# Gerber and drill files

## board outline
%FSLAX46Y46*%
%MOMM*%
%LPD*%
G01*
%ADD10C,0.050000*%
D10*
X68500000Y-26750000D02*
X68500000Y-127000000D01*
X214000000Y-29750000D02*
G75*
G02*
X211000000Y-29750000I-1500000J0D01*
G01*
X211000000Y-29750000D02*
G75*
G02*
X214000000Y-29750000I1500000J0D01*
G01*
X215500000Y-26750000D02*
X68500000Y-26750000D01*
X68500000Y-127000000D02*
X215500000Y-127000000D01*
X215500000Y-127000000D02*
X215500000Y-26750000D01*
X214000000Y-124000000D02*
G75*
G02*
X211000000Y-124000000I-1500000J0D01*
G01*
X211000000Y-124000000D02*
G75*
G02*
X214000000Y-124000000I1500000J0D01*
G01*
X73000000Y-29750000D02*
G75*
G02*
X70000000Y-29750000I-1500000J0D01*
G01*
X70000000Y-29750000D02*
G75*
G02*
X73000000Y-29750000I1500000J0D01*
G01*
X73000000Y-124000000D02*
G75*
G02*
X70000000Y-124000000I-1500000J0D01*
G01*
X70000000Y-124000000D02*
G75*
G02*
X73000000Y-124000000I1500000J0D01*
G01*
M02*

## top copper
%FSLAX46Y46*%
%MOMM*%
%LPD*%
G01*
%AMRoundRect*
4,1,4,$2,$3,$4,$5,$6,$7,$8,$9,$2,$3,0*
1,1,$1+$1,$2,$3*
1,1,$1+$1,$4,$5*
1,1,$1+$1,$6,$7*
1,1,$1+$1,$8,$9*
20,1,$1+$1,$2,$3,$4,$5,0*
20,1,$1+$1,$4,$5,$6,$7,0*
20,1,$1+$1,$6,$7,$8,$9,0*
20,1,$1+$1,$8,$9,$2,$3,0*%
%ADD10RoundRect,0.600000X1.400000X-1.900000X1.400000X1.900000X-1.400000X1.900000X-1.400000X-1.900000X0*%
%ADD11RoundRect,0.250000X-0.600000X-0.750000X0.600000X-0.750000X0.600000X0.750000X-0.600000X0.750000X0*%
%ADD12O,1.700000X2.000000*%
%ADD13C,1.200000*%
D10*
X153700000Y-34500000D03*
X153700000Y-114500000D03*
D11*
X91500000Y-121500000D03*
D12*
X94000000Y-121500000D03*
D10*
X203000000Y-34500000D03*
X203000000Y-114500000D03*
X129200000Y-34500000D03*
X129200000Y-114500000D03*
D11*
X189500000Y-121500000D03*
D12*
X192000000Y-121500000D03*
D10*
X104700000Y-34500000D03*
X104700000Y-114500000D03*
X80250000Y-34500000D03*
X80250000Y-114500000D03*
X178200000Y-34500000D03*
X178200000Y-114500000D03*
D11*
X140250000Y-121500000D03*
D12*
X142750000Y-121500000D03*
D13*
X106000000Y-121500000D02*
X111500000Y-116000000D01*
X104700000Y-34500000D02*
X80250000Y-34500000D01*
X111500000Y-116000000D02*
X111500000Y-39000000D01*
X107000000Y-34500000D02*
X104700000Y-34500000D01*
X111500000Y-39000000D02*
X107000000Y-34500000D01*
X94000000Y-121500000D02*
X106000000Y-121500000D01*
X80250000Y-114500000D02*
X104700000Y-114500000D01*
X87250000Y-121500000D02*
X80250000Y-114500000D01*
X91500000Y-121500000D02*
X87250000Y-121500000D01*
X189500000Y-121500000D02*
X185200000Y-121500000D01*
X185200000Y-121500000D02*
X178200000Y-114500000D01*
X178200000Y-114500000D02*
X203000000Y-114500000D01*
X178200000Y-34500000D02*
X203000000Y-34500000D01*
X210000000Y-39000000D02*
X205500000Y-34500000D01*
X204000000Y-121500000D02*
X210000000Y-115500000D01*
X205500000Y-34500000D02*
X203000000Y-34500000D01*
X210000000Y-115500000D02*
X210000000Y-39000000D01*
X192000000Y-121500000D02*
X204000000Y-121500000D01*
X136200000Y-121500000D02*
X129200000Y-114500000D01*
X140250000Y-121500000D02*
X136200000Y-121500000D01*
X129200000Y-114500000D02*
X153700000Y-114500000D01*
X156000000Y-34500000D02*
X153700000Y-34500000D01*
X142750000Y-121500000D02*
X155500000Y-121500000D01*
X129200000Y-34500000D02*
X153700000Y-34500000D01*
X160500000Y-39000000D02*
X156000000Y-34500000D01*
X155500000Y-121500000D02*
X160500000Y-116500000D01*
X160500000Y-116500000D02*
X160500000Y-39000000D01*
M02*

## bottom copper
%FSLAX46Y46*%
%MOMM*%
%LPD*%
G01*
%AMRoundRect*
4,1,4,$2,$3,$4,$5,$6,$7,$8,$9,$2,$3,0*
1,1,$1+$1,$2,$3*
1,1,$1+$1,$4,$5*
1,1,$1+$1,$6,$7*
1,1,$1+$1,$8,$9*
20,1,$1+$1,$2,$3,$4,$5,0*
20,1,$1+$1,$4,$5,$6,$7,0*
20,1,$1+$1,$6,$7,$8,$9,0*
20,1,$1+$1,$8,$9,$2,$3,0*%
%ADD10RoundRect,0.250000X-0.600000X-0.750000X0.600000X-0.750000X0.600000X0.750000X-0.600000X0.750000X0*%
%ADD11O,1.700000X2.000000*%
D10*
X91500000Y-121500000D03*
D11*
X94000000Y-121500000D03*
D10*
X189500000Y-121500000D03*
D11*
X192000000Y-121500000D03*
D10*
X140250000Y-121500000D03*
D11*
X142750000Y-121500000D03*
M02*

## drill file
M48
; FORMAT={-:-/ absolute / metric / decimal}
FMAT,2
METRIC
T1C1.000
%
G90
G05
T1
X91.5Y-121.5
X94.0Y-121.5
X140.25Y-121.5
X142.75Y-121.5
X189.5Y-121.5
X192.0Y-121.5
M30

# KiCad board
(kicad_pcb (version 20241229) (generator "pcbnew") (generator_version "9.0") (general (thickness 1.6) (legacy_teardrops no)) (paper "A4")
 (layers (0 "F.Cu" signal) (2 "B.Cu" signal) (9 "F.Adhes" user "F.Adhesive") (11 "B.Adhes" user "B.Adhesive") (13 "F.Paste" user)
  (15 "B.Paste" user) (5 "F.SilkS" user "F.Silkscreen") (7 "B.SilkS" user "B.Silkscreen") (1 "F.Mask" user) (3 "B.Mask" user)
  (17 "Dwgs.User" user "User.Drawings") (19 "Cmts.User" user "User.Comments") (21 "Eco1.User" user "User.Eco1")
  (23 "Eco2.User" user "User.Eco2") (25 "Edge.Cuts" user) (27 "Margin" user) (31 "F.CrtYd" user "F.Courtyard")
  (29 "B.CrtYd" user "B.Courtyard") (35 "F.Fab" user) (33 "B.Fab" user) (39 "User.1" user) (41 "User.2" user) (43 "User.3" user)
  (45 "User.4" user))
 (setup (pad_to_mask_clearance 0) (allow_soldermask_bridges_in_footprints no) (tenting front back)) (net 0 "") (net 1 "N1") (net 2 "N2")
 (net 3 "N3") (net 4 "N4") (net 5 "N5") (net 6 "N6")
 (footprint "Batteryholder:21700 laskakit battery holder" (layer "F.Cu") (at 153.7 79.5)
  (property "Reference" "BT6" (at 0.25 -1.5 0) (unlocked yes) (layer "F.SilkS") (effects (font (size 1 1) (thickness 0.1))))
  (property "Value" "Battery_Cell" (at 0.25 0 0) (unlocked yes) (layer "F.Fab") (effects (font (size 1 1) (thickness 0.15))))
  (pad "1" smd roundrect (at 0 -45 90) (size 5 4) (layers "F.Cu" "F.Mask" "F.Paste") (roundrect_rratio 0.15) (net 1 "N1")
   (thermal_bridge_angle 45))
  (pad "2" smd roundrect (at 0 35 90) (size 5 4) (layers "F.Cu" "F.Mask" "F.Paste") (roundrect_rratio 0.15) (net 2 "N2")
   (thermal_bridge_angle 45)))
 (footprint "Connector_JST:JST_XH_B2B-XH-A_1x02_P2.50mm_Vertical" (layer "F.Cu") (at 91.5 121.5)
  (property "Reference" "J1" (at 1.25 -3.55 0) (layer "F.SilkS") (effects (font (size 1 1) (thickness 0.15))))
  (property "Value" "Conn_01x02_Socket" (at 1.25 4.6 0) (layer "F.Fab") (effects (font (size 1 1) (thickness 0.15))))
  (pad "1" thru_hole roundrect (at 0 0) (size 1.7 2) (drill 1) (layers "*.Cu" "*.Mask") (remove_unused_layers no)
   (roundrect_rratio 0.147059) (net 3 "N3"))
  (pad "2" thru_hole oval (at 2.5 0) (size 1.7 2) (drill 1) (layers "*.Cu" "*.Mask") (remove_unused_layers no) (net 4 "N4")))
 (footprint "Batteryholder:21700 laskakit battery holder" (layer "F.Cu") (at 203 79.5)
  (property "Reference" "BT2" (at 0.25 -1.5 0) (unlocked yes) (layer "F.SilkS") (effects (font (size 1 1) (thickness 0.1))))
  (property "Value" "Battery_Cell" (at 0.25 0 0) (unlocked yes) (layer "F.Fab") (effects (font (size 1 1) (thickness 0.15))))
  (pad "1" smd roundrect (at 0 -45 90) (size 5 4) (layers "F.Cu" "F.Mask" "F.Paste") (roundrect_rratio 0.15) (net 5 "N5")
   (thermal_bridge_angle 45))
  (pad "2" smd roundrect (at 0 35 90) (size 5 4) (layers "F.Cu" "F.Mask" "F.Paste") (roundrect_rratio 0.15) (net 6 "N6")
   (thermal_bridge_angle 45)))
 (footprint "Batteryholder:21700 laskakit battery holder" (layer "F.Cu") (at 129.2 79.5)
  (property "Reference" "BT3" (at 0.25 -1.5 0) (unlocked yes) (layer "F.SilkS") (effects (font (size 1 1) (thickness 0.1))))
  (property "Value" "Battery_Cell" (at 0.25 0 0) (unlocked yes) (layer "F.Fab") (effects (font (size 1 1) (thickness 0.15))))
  (pad "1" smd roundrect (at 0 -45 90) (size 5 4) (layers "F.Cu" "F.Mask" "F.Paste") (roundrect_rratio 0.15) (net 1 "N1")
   (thermal_bridge_angle 45))
  (pad "2" smd roundrect (at 0 35 90) (size 5 4) (layers "F.Cu" "F.Mask" "F.Paste") (roundrect_rratio 0.15) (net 2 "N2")
   (thermal_bridge_angle 45)))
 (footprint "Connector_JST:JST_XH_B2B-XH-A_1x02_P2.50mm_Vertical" (layer "F.Cu") (at 189.5 121.5)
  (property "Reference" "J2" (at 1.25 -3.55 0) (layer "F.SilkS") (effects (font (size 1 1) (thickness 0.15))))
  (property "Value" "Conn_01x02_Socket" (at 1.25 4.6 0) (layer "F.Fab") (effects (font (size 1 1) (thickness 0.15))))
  (pad "1" thru_hole roundrect (at 0 0) (size 1.7 2) (drill 1) (layers "*.Cu" "*.Mask") (remove_unused_layers no)
   (roundrect_rratio 0.147059) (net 6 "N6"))
  (pad "2" thru_hole oval (at 2.5 0) (size 1.7 2) (drill 1) (layers "*.Cu" "*.Mask") (remove_unused_layers no) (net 5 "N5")))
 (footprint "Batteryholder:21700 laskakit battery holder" (layer "F.Cu") (at 104.7 79.5)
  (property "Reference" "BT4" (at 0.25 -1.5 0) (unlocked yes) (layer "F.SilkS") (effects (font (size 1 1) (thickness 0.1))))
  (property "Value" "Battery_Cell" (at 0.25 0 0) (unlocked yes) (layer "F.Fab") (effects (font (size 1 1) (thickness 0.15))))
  (pad "1" smd roundrect (at 0 -45 90) (size 5 4) (layers "F.Cu" "F.Mask" "F.Paste") (roundrect_rratio 0.15) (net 4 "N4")
   (thermal_bridge_angle 45))
  (pad "2" smd roundrect (at 0 35 90) (size 5 4) (layers "F.Cu" "F.Mask" "F.Paste") (roundrect_rratio 0.15) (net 3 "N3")
   (thermal_bridge_angle 45)))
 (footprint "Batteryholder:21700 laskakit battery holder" (layer "F.Cu") (at 80.25 79.5)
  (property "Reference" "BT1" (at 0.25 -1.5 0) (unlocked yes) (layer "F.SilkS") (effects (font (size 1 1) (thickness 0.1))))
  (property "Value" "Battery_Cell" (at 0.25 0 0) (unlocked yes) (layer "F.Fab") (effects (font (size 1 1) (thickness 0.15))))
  (pad "1" smd roundrect (at 0 -45 90) (size 5 4) (layers "F.Cu" "F.Mask" "F.Paste") (roundrect_rratio 0.15) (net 4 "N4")
   (thermal_bridge_angle 45))
  (pad "2" smd roundrect (at 0 35 90) (size 5 4) (layers "F.Cu" "F.Mask" "F.Paste") (roundrect_rratio 0.15) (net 3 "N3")
   (thermal_bridge_angle 45)))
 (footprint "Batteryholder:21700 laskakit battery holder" (layer "F.Cu") (at 178.2 79.5)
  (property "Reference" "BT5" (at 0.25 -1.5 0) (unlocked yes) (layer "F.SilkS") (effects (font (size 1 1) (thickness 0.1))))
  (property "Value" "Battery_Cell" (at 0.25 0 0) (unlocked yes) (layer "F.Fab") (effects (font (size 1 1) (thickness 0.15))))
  (pad "1" smd roundrect (at 0 -45 90) (size 5 4) (layers "F.Cu" "F.Mask" "F.Paste") (roundrect_rratio 0.15) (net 5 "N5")
   (thermal_bridge_angle 45))
  (pad "2" smd roundrect (at 0 35 90) (size 5 4) (layers "F.Cu" "F.Mask" "F.Paste") (roundrect_rratio 0.15) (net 6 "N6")
   (thermal_bridge_angle 45)))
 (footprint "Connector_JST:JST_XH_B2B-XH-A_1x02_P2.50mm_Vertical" (layer "F.Cu") (at 140.25 121.5)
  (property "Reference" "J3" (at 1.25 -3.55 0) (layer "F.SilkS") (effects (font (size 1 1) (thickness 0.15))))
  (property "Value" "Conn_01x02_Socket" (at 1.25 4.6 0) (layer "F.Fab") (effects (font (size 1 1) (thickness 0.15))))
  (pad "1" thru_hole roundrect (at 0 0) (size 1.7 2) (drill 1) (layers "*.Cu" "*.Mask") (remove_unused_layers no)
   (roundrect_rratio 0.147059) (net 2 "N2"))
  (pad "2" thru_hole oval (at 2.5 0) (size 1.7 2) (drill 1) (layers "*.Cu" "*.Mask") (remove_unused_layers no) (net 1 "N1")))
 (gr_line (start 68.5 26.75) (end 68.5 127) (stroke (width 0.05) (type default)) (layer "Edge.Cuts"))
 (gr_circle (center 212.5 29.75) (end 214 29.75) (stroke (width 0.05) (type default)) (fill no) (layer "Edge.Cuts"))
 (gr_line (start 215.5 26.75) (end 68.5 26.75) (stroke (width 0.05) (type default)) (layer "Edge.Cuts"))
 (gr_line (start 68.5 127) (end 215.5 127) (stroke (width 0.05) (type default)) (layer "Edge.Cuts"))
 (gr_line (start 215.5 127) (end 215.5 26.75) (stroke (width 0.05) (type default)) (layer "Edge.Cuts"))
 (gr_circle (center 212.5 124) (end 214 124) (stroke (width 0.05) (type default)) (fill no) (layer "Edge.Cuts"))
 (gr_circle (center 71.5 29.75) (end 73 29.75) (stroke (width 0.05) (type default)) (fill no) (layer "Edge.Cuts"))
 (gr_circle (center 71.5 124) (end 73 124) (stroke (width 0.05) (type default)) (fill no) (layer "Edge.Cuts"))
 (segment (start 106 121.5) (end 111.5 116) (width 1.2) (layer "F.Cu") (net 4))
 (segment (start 104.7 34.5) (end 80.25 34.5) (width 1.2) (layer "F.Cu") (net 4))
 (segment (start 111.5 116) (end 111.5 39) (width 1.2) (layer "F.Cu") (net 4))
 (segment (start 107 34.5) (end 104.7 34.5) (width 1.2) (layer "F.Cu") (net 4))
 (segment (start 111.5 39) (end 107 34.5) (width 1.2) (layer "F.Cu") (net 4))
 (segment (start 94 121.5) (end 106 121.5) (width 1.2) (layer "F.Cu") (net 4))
 (segment (start 80.25 114.5) (end 104.7 114.5) (width 1.2) (layer "F.Cu") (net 3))
 (segment (start 87.25 121.5) (end 80.25 114.5) (width 1.2) (layer "F.Cu") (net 3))
 (segment (start 91.5 121.5) (end 87.25 121.5) (width 1.2) (layer "F.Cu") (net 3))
 (segment (start 189.5 121.5) (end 185.2 121.5) (width 1.2) (layer "F.Cu") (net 6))
 (segment (start 185.2 121.5) (end 178.2 114.5) (width 1.2) (layer "F.Cu") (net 6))
 (segment (start 178.2 114.5) (end 203 114.5) (width 1.2) (layer "F.Cu") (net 6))
 (segment (start 178.2 34.5) (end 203 34.5) (width 1.2) (layer "F.Cu") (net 5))
 (segment (start 210 39) (end 205.5 34.5) (width 1.2) (layer "F.Cu") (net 5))
 (segment (start 204 121.5) (end 210 115.5) (width 1.2) (layer "F.Cu") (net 5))
 (segment (start 205.5 34.5) (end 203 34.5) (width 1.2) (layer "F.Cu") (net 5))
 (segment (start 210 115.5) (end 210 39) (width 1.2) (layer "F.Cu") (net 5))
 (segment (start 192 121.5) (end 204 121.5) (width 1.2) (layer "F.Cu") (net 5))
 (segment (start 136.2 121.5) (end 129.2 114.5) (width 1.2) (layer "F.Cu") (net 2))
 (segment (start 140.25 121.5) (end 136.2 121.5) (width 1.2) (layer "F.Cu") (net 2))
 (segment (start 129.2 114.5) (end 153.7 114.5) (width 1.2) (layer "F.Cu") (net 2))
 (segment (start 156 34.5) (end 153.7 34.5) (width 1.2) (layer "F.Cu") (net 1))
 (segment (start 142.75 121.5) (end 155.5 121.5) (width 1.2) (layer "F.Cu") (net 1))
 (segment (start 129.2 34.5) (end 153.7 34.5) (width 1.2) (layer "F.Cu") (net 1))
 (segment (start 160.5 39) (end 156 34.5) (width 1.2) (layer "F.Cu") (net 1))
 (segment (start 155.5 121.5) (end 160.5 116.5) (width 1.2) (layer "F.Cu") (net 1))
 (segment (start 160.5 116.5) (end 160.5 39) (width 1.2) (layer "F.Cu") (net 1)))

